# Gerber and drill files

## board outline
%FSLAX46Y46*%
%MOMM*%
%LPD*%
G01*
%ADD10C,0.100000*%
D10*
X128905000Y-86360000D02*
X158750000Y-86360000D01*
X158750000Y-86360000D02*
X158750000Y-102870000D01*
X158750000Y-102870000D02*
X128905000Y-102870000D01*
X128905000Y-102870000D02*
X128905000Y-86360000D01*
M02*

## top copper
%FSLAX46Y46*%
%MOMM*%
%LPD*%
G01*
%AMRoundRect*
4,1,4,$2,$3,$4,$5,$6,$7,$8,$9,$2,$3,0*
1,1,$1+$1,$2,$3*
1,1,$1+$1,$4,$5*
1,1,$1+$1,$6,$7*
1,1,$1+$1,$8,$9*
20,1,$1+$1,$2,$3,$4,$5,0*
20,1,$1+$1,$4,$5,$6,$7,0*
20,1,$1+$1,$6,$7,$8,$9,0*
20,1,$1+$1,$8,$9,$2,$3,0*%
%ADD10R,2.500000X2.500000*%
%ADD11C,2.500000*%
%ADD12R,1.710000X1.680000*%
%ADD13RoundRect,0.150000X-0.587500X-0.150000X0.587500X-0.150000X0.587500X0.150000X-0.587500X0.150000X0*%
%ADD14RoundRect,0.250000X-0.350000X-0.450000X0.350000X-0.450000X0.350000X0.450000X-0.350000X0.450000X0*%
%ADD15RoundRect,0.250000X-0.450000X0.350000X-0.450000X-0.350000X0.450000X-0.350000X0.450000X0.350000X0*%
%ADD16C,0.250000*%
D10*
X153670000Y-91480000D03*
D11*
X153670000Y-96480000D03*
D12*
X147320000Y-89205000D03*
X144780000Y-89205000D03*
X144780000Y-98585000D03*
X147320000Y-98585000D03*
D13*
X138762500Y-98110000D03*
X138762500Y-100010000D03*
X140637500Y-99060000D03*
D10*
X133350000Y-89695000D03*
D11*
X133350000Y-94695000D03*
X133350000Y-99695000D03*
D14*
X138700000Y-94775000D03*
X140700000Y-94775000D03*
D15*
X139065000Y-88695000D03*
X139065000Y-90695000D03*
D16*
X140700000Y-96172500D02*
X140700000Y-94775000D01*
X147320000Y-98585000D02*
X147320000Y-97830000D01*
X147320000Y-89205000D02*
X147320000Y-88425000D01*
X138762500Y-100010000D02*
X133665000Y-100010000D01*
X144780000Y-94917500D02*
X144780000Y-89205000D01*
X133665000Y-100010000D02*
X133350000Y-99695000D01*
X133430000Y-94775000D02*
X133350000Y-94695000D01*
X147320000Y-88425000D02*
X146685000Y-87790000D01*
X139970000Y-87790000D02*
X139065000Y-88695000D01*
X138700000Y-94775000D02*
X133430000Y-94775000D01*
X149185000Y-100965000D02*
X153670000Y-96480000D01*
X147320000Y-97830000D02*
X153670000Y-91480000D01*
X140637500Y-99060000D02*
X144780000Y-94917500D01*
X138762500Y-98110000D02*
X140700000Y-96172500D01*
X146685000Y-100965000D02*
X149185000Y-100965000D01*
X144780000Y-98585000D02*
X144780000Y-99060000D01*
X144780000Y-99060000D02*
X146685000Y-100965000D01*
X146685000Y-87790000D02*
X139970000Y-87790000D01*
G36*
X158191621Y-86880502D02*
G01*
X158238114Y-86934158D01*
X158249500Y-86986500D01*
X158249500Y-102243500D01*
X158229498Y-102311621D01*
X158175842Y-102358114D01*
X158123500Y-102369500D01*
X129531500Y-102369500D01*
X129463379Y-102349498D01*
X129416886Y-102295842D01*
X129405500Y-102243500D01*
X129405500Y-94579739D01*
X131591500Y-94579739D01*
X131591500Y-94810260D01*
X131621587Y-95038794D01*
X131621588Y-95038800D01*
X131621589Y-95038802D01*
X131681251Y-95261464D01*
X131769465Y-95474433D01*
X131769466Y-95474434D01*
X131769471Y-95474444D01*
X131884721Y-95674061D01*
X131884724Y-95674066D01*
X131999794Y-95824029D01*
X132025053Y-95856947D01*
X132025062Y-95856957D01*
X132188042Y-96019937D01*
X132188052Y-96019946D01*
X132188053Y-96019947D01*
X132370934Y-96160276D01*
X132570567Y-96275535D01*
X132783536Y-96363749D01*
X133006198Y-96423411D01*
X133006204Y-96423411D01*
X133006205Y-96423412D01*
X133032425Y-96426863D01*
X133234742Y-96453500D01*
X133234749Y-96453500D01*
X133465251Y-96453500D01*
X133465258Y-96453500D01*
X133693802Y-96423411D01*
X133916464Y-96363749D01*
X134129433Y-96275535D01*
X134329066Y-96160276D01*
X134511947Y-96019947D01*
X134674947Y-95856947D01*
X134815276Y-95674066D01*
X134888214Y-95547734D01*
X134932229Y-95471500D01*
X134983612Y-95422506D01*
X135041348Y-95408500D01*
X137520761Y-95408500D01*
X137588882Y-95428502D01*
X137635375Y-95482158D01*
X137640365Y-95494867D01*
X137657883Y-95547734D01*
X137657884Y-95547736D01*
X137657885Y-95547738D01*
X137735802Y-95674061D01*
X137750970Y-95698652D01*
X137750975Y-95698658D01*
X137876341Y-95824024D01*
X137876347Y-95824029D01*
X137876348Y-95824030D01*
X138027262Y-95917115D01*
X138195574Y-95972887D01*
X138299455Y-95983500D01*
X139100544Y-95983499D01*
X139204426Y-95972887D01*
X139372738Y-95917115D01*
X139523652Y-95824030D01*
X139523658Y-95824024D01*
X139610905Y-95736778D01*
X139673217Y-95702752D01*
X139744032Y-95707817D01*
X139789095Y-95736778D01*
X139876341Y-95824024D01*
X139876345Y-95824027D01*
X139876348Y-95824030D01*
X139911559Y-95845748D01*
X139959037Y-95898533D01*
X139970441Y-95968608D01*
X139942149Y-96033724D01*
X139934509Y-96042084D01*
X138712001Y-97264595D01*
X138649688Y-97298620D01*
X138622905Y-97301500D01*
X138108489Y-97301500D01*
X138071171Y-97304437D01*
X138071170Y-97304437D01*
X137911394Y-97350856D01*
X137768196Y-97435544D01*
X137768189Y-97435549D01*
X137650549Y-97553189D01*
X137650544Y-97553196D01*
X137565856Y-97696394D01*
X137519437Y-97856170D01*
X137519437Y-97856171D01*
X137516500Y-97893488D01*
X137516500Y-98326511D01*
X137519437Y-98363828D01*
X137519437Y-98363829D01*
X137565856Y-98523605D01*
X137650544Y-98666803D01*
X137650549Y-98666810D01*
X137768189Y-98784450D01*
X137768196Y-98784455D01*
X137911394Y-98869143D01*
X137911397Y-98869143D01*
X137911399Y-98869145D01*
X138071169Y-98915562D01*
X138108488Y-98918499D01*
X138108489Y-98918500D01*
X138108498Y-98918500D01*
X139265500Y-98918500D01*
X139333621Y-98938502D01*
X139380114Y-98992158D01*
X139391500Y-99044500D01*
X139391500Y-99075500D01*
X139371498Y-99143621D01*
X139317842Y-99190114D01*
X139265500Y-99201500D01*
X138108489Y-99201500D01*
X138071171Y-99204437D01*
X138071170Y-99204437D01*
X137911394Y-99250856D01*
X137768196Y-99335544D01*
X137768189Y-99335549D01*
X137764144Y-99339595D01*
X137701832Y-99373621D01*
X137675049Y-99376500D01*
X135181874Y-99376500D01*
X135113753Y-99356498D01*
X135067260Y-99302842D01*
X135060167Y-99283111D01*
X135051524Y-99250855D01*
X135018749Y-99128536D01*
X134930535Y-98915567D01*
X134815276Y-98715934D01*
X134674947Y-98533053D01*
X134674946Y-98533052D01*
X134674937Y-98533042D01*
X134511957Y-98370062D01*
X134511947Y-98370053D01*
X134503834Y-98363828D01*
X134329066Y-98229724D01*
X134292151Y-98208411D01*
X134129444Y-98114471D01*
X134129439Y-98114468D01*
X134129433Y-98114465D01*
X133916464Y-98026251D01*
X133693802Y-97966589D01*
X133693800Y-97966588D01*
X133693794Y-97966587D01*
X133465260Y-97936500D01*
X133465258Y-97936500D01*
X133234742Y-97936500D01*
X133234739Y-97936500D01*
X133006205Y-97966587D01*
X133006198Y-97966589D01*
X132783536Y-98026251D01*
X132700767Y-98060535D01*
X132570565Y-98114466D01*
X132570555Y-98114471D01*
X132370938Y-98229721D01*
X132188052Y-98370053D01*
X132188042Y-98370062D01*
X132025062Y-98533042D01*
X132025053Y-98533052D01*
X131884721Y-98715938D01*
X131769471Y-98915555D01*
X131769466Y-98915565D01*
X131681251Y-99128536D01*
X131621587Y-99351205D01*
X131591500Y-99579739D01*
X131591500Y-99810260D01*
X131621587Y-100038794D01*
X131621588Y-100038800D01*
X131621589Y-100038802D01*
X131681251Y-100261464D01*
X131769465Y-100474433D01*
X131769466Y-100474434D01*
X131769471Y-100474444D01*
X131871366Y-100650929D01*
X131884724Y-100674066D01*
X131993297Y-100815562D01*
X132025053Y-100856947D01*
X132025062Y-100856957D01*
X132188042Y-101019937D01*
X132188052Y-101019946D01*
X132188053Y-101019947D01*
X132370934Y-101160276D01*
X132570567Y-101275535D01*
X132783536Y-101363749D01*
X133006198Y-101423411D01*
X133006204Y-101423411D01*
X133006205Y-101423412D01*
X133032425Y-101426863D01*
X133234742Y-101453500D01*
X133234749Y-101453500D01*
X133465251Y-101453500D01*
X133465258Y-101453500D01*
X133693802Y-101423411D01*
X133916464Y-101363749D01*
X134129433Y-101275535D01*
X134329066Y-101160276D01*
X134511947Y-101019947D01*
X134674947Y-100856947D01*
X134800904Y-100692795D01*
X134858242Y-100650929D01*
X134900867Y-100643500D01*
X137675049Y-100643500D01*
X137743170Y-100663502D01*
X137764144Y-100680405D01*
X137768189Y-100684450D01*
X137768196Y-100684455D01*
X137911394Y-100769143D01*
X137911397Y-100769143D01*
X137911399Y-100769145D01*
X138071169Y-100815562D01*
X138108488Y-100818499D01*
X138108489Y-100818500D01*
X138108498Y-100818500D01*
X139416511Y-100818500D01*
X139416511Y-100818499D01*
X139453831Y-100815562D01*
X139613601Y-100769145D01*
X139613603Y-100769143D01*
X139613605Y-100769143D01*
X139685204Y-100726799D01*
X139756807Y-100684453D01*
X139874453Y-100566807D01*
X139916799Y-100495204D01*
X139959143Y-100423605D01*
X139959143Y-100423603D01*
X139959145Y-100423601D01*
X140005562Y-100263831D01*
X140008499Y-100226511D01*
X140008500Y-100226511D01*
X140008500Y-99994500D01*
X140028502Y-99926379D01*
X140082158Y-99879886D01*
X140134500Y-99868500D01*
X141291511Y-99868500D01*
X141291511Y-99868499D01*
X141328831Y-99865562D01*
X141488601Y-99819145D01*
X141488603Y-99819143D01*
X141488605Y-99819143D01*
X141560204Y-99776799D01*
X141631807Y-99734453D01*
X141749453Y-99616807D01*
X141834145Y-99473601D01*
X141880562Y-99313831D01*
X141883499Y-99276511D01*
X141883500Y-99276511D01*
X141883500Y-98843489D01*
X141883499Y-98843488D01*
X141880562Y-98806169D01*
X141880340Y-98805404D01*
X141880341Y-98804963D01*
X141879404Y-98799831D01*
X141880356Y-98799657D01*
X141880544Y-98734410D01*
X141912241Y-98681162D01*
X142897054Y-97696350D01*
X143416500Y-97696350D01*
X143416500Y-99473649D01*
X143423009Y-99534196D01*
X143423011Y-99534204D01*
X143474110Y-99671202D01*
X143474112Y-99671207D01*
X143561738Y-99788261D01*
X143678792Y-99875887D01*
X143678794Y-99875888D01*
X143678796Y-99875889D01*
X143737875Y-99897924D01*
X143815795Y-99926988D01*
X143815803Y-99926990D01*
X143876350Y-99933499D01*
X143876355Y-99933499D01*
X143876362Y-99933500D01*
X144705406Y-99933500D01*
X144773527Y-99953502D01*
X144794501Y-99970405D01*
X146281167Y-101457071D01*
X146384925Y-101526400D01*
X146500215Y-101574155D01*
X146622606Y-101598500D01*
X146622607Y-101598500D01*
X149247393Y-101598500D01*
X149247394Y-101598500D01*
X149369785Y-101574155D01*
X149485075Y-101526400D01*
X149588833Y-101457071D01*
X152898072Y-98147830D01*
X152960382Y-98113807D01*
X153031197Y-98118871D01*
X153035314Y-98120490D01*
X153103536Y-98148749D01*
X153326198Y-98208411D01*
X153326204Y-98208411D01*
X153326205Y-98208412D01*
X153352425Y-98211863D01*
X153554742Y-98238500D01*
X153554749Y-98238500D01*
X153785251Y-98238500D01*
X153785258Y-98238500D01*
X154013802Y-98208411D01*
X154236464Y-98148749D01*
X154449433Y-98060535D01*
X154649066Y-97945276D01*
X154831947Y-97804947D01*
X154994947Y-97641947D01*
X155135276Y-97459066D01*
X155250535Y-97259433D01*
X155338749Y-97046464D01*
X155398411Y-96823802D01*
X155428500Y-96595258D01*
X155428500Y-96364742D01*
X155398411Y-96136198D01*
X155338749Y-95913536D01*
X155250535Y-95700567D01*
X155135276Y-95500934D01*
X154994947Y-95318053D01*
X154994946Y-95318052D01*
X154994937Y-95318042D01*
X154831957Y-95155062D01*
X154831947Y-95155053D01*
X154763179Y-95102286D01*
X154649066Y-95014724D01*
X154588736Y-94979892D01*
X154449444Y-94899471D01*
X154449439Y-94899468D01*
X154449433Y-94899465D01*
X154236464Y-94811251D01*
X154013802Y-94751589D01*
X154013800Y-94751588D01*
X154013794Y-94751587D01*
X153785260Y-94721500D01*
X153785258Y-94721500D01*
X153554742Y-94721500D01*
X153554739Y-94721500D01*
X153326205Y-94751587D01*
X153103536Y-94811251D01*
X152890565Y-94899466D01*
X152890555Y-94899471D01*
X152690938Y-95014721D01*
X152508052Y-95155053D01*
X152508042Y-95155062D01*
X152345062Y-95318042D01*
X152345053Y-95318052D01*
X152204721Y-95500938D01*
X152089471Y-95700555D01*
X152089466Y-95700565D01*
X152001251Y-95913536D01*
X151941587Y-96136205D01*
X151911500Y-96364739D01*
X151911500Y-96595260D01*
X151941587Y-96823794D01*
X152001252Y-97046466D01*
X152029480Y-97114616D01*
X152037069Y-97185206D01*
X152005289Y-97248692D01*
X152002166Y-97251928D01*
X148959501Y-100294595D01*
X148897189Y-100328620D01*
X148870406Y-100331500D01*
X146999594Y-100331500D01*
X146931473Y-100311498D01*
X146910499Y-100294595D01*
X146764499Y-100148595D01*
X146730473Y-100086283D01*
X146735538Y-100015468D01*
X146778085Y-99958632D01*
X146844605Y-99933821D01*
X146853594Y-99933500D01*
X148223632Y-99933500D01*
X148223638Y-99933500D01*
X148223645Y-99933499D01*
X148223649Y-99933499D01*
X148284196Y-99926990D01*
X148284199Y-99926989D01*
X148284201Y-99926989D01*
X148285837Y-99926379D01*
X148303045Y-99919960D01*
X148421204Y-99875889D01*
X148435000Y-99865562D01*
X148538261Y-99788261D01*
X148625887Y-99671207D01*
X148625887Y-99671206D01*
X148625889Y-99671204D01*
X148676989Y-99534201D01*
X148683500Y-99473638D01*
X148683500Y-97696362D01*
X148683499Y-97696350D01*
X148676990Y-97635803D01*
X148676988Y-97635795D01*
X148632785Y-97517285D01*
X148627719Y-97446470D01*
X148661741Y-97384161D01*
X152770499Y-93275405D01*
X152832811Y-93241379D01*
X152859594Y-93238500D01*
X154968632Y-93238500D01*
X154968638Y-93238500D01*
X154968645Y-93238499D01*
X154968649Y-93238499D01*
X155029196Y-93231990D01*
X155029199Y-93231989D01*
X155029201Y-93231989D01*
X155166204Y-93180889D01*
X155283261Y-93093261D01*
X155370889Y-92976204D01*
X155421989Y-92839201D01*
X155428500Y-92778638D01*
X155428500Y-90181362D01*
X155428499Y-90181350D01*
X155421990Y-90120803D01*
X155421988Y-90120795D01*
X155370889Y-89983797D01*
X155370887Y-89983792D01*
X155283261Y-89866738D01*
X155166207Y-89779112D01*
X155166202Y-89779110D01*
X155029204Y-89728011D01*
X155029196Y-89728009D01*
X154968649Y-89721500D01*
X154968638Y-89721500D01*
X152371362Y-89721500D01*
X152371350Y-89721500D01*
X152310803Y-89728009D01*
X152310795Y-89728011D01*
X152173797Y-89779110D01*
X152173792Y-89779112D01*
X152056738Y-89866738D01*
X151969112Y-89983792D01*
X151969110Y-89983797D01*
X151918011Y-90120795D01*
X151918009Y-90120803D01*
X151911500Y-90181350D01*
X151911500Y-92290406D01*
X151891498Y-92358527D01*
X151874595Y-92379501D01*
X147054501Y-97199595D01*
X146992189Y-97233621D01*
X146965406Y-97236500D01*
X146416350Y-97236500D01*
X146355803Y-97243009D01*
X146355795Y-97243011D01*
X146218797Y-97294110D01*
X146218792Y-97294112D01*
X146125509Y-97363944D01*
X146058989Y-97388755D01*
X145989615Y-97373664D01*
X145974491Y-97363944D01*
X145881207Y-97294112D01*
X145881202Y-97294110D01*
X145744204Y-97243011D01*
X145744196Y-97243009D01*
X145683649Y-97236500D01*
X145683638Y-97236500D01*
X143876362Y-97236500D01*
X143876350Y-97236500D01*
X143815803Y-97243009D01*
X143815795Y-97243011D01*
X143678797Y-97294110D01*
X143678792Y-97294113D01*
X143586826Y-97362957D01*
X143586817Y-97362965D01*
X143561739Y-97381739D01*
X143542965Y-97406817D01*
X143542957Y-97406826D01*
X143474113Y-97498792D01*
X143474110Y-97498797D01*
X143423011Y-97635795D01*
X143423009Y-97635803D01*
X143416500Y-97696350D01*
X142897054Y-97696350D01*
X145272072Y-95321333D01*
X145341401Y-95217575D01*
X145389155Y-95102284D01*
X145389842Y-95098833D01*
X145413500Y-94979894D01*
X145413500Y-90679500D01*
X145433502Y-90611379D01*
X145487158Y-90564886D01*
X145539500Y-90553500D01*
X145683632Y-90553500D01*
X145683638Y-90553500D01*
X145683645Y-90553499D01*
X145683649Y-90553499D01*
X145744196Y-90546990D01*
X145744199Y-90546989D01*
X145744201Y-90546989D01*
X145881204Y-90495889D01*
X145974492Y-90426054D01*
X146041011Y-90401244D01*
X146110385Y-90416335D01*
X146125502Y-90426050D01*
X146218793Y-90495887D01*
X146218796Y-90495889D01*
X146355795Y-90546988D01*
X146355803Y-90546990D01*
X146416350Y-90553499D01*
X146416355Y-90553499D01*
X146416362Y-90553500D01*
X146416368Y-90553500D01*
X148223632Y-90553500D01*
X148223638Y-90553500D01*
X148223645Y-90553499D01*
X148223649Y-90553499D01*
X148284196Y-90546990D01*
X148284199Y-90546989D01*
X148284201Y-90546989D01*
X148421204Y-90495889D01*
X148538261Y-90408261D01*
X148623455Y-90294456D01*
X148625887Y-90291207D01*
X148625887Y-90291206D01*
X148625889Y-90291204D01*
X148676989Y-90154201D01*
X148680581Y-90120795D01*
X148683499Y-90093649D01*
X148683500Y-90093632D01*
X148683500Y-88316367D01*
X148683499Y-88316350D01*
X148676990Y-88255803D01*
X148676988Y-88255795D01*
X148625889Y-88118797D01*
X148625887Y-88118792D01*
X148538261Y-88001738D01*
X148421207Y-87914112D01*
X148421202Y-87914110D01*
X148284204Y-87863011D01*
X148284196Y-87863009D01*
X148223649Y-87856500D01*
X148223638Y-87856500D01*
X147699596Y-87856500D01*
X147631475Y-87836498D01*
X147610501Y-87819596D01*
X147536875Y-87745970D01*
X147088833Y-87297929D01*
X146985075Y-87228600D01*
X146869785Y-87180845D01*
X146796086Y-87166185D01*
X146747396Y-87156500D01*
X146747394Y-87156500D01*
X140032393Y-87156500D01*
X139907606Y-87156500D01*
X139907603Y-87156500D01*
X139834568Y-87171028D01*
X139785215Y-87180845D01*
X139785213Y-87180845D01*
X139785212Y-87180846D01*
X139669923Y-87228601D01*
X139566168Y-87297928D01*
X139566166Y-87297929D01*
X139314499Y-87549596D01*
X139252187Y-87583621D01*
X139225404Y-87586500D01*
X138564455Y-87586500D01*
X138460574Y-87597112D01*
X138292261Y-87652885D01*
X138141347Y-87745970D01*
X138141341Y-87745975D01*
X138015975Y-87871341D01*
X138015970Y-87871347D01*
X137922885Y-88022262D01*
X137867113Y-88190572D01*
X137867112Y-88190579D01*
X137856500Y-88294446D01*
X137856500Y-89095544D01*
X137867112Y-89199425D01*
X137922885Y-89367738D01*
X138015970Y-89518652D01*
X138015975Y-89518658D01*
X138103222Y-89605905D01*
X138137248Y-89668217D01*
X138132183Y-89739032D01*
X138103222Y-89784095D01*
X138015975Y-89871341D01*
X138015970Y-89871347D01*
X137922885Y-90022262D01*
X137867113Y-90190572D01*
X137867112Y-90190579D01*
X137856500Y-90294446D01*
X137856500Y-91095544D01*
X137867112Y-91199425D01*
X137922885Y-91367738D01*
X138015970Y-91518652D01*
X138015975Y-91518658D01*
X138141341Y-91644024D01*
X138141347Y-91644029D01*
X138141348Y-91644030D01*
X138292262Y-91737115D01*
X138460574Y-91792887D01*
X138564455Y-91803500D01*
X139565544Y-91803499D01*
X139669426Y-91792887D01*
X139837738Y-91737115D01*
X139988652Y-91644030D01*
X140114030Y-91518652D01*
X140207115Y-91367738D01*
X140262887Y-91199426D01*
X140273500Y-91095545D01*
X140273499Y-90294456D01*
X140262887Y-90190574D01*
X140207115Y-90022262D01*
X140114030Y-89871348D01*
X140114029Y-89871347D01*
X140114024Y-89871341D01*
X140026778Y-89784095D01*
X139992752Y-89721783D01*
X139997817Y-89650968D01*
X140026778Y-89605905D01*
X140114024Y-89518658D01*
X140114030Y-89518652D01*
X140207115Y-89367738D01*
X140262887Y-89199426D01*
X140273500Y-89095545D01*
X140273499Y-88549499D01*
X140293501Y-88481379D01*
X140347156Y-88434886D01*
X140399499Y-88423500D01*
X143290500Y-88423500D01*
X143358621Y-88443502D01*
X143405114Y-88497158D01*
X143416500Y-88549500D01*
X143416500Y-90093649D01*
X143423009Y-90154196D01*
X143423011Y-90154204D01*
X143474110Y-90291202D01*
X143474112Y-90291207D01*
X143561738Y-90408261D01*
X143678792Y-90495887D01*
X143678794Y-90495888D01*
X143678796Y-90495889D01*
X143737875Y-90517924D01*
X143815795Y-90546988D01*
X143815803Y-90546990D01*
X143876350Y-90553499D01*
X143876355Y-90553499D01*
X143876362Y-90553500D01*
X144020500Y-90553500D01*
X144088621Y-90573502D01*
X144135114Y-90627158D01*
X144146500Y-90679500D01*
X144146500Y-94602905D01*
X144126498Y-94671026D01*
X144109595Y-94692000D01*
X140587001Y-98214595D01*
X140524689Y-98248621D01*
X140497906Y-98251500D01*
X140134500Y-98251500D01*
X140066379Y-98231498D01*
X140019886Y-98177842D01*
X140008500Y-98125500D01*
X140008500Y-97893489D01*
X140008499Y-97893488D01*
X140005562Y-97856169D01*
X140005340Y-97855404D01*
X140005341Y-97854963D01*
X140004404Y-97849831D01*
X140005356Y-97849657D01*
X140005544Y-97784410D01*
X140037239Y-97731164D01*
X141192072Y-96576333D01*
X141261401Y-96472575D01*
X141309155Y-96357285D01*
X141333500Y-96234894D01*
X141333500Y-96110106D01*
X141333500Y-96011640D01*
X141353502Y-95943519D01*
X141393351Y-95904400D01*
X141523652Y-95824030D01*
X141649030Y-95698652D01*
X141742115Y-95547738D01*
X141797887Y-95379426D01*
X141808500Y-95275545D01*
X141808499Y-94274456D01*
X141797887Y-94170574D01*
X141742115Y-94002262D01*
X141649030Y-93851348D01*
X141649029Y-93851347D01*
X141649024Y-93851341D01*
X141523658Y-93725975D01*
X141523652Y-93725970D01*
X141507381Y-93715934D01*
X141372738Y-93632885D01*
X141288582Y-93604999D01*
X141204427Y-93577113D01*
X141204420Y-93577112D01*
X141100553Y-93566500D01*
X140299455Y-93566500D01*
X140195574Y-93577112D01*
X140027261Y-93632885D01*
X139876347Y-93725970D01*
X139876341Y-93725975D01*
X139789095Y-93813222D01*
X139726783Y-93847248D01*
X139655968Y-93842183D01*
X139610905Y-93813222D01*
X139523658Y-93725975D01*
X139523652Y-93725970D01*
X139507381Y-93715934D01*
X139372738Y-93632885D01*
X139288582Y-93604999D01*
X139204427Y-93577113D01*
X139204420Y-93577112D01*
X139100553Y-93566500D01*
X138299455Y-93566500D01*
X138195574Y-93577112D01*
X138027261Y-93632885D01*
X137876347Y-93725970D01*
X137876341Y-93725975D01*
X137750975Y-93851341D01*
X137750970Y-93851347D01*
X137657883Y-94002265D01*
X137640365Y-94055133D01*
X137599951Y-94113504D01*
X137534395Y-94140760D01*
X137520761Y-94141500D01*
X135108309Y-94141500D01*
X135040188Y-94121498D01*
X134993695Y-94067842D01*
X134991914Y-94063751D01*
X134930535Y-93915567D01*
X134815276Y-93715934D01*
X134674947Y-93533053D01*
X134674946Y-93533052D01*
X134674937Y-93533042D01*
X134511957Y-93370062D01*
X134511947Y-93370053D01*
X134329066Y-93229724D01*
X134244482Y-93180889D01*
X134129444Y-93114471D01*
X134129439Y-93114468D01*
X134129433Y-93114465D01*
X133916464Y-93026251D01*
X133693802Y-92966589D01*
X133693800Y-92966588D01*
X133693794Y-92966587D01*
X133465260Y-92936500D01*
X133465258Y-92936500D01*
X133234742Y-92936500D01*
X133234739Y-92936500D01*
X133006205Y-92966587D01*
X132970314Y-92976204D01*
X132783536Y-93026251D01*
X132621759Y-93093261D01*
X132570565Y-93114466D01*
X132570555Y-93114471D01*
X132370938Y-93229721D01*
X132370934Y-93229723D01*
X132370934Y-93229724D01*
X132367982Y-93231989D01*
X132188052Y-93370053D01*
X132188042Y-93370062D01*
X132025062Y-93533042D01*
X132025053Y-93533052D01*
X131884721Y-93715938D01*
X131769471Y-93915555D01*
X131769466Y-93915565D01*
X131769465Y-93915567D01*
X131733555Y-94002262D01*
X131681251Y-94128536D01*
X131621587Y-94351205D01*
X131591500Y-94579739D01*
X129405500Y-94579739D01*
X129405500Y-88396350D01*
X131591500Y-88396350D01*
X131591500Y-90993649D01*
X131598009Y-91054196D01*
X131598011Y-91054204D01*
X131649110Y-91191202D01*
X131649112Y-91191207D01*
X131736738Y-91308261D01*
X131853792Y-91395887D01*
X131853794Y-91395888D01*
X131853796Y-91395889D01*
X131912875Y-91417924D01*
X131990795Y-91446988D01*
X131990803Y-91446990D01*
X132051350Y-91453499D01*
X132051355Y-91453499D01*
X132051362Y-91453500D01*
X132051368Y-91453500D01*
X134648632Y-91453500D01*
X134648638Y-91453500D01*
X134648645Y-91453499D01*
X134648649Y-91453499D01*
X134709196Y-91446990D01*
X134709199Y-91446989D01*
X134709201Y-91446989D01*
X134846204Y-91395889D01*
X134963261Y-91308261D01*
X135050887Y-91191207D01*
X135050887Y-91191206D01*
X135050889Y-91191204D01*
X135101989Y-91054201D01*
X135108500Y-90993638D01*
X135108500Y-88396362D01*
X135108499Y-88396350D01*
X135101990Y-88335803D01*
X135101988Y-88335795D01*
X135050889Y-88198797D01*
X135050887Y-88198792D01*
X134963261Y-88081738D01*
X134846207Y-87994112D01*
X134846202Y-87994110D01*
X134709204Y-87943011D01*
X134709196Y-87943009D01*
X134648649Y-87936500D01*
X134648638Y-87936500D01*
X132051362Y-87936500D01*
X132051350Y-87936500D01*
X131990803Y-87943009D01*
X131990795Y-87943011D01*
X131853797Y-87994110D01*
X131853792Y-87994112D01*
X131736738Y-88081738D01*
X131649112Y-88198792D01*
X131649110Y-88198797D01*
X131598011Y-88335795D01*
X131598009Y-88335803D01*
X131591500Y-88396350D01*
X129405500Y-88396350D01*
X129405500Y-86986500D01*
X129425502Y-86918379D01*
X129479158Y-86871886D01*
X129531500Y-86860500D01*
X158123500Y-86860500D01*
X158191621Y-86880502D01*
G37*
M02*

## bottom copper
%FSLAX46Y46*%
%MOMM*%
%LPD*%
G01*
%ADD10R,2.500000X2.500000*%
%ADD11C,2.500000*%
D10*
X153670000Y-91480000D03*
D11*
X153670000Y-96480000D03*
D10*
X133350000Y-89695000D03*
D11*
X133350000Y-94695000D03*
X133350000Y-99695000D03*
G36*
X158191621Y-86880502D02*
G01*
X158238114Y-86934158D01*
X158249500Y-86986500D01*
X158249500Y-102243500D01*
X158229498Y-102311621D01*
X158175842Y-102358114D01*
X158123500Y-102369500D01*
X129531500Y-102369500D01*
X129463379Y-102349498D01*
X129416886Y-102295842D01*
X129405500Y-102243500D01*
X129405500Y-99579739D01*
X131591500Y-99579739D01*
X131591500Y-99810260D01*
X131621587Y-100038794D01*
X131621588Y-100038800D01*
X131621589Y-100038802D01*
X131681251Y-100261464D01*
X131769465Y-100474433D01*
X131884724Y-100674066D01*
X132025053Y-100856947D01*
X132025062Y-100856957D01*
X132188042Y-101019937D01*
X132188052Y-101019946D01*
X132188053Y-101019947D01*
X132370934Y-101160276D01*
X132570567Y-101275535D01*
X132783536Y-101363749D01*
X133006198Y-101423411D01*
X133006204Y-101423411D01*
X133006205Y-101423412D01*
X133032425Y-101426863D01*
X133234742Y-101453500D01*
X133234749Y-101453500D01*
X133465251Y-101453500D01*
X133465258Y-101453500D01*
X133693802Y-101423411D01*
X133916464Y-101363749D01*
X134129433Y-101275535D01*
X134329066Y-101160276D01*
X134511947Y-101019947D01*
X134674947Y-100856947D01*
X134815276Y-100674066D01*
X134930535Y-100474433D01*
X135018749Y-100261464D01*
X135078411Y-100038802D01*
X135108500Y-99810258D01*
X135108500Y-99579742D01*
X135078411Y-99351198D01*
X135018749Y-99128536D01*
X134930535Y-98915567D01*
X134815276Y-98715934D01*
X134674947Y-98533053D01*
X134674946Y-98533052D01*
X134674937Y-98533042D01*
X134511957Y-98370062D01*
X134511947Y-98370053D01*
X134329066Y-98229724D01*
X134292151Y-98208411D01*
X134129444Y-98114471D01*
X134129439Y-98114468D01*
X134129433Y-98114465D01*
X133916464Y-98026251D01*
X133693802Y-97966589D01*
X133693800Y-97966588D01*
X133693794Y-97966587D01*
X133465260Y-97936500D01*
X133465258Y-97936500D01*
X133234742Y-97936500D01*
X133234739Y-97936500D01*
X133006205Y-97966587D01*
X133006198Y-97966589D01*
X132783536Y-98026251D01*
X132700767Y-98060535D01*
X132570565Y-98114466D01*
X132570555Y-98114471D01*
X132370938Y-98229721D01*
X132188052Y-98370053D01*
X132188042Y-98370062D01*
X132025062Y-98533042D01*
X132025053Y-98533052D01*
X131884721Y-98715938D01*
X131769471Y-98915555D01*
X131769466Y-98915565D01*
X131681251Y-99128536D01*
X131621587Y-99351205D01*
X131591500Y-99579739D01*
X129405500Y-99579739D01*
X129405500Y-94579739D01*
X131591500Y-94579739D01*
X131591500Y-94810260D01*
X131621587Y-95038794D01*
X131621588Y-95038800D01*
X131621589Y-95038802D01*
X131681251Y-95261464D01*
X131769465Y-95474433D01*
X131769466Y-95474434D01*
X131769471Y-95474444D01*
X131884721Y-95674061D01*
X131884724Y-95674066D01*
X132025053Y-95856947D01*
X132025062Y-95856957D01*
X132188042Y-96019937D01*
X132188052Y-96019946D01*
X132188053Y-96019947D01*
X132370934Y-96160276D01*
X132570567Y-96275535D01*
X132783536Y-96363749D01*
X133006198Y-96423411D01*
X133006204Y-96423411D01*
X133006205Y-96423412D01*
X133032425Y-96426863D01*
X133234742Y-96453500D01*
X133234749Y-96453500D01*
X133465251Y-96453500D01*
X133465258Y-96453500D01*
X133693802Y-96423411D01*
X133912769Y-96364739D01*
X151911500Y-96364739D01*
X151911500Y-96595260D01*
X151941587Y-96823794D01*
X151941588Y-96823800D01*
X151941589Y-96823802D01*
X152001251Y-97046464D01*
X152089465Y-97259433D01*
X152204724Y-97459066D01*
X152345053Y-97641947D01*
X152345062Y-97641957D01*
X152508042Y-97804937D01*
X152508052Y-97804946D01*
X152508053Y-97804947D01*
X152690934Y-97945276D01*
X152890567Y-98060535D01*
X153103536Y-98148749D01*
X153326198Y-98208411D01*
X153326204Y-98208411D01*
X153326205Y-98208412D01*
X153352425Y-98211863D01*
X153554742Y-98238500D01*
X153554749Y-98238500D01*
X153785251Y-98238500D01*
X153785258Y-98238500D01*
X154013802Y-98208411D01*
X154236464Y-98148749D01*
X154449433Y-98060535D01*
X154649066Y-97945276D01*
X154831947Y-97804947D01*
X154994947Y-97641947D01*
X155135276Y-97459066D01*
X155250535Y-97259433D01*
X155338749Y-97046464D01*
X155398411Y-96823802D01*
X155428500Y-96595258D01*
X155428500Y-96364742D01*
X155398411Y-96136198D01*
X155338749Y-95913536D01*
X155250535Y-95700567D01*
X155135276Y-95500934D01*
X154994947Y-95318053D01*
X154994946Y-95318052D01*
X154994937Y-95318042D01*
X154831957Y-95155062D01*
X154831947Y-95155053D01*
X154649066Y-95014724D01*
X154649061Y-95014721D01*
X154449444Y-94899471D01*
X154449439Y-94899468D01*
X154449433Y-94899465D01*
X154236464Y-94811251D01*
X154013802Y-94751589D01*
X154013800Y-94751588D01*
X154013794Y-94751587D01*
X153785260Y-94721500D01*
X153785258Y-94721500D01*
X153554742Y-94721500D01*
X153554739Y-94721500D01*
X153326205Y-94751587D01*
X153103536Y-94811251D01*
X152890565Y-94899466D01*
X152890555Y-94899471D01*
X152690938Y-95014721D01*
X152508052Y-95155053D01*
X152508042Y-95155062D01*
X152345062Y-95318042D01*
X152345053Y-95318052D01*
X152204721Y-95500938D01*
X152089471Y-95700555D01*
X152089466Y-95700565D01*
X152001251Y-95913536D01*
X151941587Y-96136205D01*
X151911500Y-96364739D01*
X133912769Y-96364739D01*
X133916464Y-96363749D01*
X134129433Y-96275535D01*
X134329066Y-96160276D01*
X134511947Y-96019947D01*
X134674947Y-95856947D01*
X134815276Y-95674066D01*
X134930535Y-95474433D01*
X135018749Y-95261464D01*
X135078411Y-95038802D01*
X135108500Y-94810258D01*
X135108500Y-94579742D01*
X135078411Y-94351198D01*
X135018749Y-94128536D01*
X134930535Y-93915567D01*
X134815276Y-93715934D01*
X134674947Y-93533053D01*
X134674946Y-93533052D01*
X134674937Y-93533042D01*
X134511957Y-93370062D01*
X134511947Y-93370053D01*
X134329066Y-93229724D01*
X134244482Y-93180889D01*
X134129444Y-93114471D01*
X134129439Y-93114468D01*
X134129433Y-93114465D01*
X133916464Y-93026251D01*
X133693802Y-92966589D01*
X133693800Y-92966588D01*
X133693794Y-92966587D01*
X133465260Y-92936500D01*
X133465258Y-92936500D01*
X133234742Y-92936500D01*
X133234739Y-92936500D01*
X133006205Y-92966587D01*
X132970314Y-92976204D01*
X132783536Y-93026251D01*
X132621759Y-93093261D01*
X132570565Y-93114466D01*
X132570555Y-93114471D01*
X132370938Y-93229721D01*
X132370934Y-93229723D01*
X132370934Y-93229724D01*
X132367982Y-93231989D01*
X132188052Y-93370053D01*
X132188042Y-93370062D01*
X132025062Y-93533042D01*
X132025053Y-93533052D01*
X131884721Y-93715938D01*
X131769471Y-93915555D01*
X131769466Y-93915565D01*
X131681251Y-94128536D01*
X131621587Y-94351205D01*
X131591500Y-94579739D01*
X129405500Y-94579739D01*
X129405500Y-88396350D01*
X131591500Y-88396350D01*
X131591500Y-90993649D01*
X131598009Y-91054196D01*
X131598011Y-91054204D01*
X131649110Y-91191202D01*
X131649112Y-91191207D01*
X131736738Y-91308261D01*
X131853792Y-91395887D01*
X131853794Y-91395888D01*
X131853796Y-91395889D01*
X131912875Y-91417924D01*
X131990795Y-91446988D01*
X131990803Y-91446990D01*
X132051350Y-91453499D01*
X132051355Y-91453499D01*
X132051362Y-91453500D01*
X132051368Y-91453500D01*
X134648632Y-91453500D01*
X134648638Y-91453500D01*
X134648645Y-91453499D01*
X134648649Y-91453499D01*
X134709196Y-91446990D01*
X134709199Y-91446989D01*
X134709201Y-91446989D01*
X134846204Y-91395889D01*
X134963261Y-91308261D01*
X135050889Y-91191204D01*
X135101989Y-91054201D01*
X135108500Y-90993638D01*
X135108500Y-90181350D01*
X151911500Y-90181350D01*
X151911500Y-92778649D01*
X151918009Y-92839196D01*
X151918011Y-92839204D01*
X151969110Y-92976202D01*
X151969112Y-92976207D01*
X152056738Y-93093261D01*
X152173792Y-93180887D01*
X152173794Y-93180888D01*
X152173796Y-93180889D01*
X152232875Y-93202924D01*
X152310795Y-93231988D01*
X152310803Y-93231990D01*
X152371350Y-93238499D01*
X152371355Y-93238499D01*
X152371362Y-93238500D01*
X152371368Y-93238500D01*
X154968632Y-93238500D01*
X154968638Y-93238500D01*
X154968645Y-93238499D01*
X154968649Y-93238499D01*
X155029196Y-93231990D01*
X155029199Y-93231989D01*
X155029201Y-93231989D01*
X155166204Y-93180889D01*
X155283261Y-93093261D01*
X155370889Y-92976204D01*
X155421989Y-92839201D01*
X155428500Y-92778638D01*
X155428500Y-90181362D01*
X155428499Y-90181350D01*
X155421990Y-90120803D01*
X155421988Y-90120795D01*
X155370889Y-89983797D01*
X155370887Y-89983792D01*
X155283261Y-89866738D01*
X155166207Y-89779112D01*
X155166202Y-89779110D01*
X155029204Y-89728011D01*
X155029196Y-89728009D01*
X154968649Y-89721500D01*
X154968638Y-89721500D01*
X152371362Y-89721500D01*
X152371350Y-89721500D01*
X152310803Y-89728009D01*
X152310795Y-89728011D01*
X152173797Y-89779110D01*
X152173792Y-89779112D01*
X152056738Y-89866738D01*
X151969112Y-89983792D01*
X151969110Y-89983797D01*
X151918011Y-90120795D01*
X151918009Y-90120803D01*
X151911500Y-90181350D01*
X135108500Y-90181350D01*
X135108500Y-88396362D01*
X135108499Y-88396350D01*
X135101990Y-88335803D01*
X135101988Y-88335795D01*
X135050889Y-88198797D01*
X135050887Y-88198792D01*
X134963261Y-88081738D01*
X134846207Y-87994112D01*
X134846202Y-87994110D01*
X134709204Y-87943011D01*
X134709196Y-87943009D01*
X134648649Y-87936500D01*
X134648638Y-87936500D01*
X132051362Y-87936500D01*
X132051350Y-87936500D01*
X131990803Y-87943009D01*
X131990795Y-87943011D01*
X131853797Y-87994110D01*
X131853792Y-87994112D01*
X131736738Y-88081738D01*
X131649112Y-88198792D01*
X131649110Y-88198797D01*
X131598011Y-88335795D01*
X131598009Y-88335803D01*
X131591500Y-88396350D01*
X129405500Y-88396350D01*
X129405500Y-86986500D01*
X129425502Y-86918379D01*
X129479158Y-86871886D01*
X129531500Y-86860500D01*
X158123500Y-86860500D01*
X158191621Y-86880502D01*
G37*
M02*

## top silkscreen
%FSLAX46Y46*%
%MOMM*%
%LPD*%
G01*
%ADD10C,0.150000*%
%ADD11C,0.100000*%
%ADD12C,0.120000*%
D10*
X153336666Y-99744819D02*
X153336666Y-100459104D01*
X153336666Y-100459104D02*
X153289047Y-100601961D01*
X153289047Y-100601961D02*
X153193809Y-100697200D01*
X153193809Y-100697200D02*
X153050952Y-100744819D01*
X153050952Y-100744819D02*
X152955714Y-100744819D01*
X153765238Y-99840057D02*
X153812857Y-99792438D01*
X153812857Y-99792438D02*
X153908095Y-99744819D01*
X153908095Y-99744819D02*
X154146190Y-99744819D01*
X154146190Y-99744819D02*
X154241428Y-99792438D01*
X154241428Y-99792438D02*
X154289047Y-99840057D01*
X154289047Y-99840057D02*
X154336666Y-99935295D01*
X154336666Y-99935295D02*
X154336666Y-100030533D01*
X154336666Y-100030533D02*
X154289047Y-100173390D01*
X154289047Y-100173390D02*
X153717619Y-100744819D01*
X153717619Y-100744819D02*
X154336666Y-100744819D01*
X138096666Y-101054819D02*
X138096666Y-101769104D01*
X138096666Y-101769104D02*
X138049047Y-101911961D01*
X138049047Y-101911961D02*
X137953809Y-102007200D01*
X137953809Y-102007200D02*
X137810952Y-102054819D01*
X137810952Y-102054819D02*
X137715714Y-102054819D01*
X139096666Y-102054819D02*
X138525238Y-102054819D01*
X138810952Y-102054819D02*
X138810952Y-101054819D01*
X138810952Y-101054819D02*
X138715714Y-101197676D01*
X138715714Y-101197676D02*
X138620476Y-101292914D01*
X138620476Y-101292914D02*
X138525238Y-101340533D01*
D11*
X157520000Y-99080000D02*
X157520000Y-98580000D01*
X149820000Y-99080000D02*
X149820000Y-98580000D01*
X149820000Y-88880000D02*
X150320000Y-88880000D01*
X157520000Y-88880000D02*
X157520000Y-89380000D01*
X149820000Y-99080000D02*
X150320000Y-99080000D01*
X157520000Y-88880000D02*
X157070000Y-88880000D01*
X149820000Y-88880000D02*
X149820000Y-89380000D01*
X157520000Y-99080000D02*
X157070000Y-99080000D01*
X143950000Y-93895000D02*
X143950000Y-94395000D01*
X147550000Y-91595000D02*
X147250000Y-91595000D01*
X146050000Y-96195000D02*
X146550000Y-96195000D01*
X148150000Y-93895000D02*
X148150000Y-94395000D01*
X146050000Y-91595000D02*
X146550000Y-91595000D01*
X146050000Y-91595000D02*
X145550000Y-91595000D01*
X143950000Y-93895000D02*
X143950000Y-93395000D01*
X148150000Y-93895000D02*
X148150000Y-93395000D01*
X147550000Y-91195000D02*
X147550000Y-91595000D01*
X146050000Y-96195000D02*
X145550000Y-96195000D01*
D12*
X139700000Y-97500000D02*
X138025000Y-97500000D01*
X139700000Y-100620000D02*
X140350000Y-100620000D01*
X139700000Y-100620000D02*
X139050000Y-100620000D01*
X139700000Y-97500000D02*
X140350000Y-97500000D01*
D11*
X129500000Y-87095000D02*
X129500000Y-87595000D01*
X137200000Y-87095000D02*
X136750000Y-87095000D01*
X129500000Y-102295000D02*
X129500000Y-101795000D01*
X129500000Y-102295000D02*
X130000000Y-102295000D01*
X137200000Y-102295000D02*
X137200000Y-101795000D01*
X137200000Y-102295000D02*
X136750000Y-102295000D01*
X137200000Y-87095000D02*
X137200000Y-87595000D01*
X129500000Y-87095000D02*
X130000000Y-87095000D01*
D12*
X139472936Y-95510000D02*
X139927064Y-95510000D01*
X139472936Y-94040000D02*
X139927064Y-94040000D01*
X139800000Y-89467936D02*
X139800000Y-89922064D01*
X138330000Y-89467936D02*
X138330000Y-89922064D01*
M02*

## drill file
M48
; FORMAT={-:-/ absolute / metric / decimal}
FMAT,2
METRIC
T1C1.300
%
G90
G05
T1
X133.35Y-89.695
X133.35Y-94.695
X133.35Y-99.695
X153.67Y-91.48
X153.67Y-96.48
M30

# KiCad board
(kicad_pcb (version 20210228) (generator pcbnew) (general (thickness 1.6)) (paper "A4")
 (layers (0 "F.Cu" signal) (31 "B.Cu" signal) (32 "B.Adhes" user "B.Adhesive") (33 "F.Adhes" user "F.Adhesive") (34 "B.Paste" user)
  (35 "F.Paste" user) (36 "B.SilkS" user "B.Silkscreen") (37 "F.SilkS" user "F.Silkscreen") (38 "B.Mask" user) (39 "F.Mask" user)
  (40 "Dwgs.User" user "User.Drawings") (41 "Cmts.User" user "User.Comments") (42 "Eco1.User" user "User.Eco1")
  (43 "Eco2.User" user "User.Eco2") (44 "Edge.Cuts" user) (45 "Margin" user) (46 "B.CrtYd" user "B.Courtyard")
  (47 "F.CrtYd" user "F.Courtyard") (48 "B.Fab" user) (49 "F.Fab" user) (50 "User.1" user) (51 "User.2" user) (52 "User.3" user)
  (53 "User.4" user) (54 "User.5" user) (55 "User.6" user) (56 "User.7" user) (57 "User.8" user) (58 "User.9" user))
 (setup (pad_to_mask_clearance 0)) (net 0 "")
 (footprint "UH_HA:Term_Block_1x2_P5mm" (layer "F.Cu") (at 153.67 91.48 -90)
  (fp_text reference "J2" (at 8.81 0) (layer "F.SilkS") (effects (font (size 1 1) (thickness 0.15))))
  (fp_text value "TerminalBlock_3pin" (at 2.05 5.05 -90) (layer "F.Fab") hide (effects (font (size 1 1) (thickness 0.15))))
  (fp_line (start 7.6 -3.85) (end 7.1 -3.85) (layer "F.SilkS") (width 0.1))
  (fp_line (start 7.6 3.85) (end 7.1 3.85) (layer "F.SilkS") (width 0.1))
  (fp_line (start -2.6 3.85) (end -2.6 3.35) (layer "F.SilkS") (width 0.1))
  (fp_line (start -2.6 -3.85) (end -2.1 -3.85) (layer "F.SilkS") (width 0.1))
  (fp_line (start 7.6 3.85) (end 7.6 3.35) (layer "F.SilkS") (width 0.1))
  (fp_line (start -2.6 -3.85) (end -2.6 -3.4) (layer "F.SilkS") (width 0.1))
  (fp_line (start -2.6 3.85) (end -2.1 3.85) (layer "F.SilkS") (width 0.1))
  (fp_line (start 7.6 -3.85) (end 7.6 -3.4) (layer "F.SilkS") (width 0.1))
  (pad "1" thru_hole rect (at 0 0 270) (locked) (size 2.5 2.5) (drill 1.3) (layers *.Cu *.Mask))
  (pad "2" thru_hole circle (at 5 0 270) (locked) (size 2.5 2.5) (drill 1.3) (layers *.Cu *.Mask)))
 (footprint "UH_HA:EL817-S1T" (layer "F.Cu") (at 146.05 93.895 -90)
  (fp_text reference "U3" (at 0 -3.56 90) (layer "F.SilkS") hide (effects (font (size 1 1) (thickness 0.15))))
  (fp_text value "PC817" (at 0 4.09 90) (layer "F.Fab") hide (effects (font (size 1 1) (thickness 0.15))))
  (fp_line (start 0 2.1) (end 0.5 2.1) (layer "F.SilkS") (width 0.1))
  (fp_line (start -2.3 -1.5) (end -2.3 -1.2) (layer "F.SilkS") (width 0.1))
  (fp_line (start 2.3 0) (end 2.3 -0.5) (layer "F.SilkS") (width 0.1))
  (fp_line (start 0 -2.1) (end 0.5 -2.1) (layer "F.SilkS") (width 0.1))
  (fp_line (start -2.3 0) (end -2.3 -0.5) (layer "F.SilkS") (width 0.1))
  (fp_line (start -2.3 0) (end -2.3 0.5) (layer "F.SilkS") (width 0.1))
  (fp_line (start 0 2.1) (end -0.5 2.1) (layer "F.SilkS") (width 0.1))
  (fp_line (start 0 -2.1) (end -0.5 -2.1) (layer "F.SilkS") (width 0.1))
  (fp_line (start -2.7 -1.5) (end -2.3 -1.5) (layer "F.SilkS") (width 0.1))
  (fp_line (start 2.3 0) (end 2.3 0.5) (layer "F.SilkS") (width 0.1))
  (pad "1" smd rect (at -4.69 -1.27 270) (locked) (size 1.68 1.71) (layers "F.Cu" "F.Paste" "F.Mask"))
  (pad "2" smd rect (at -4.69 1.27 270) (locked) (size 1.68 1.71) (layers "F.Cu" "F.Paste" "F.Mask"))
  (pad "3" smd rect (at 4.69 1.27 270) (locked) (size 1.68 1.71) (layers "F.Cu" "F.Paste" "F.Mask"))
  (pad "4" smd rect (at 4.69 -1.27 270) (locked) (size 1.68 1.71) (layers "F.Cu" "F.Paste" "F.Mask")))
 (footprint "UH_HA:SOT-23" (layer "F.Cu") (at 139.7 99.06)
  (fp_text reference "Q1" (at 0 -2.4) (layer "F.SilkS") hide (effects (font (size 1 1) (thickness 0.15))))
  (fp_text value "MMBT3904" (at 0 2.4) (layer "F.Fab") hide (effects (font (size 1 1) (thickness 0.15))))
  (fp_line (start 0 -1.56) (end -1.675 -1.56) (layer "F.SilkS") (width 0.12))
  (fp_line (start 0 1.56) (end 0.65 1.56) (layer "F.SilkS") (width 0.12))
  (fp_line (start 0 1.56) (end -0.65 1.56) (layer "F.SilkS") (width 0.12))
  (fp_line (start 0 -1.56) (end 0.65 -1.56) (layer "F.SilkS") (width 0.12))
  (pad "1" smd roundrect (at -0.9375 -0.95) (locked) (size 1.475 0.6) (layers "F.Cu" "F.Paste" "F.Mask") (roundrect_rratio 0.25))
  (pad "2" smd roundrect (at -0.9375 0.95) (locked) (size 1.475 0.6) (layers "F.Cu" "F.Paste" "F.Mask") (roundrect_rratio 0.25))
  (pad "3" smd roundrect (at 0.9375 0) (locked) (size 1.475 0.6) (layers "F.Cu" "F.Paste" "F.Mask") (roundrect_rratio 0.25)))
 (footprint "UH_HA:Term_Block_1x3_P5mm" (layer "F.Cu") (at 133.35 89.695 -90)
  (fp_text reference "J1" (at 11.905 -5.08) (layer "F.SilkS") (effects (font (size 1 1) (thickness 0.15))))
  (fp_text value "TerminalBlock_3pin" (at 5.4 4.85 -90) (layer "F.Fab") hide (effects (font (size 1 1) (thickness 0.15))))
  (fp_line (start -2.6 3.85) (end -2.1 3.85) (layer "F.SilkS") (width 0.1))
  (fp_line (start -2.6 -3.85) (end -2.6 -3.4) (layer "F.SilkS") (width 0.1))
  (fp_line (start 12.6 3.85) (end 12.1 3.85) (layer "F.SilkS") (width 0.1))
  (fp_line (start 12.6 3.85) (end 12.6 3.35) (layer "F.SilkS") (width 0.1))
  (fp_line (start 12.6 -3.85) (end 12.1 -3.85) (layer "F.SilkS") (width 0.1))
  (fp_line (start 12.6 -3.85) (end 12.6 -3.4) (layer "F.SilkS") (width 0.1))
  (fp_line (start -2.6 -3.85) (end -2.1 -3.85) (layer "F.SilkS") (width 0.1))
  (fp_line (start -2.6 3.85) (end -2.6 3.35) (layer "F.SilkS") (width 0.1))
  (pad "1" thru_hole rect (at 0 0 270) (locked) (size 2.5 2.5) (drill 1.3) (layers *.Cu *.Mask))
  (pad "2" thru_hole circle (at 5 0 270) (locked) (size 2.5 2.5) (drill 1.3) (layers *.Cu *.Mask))
  (pad "3" thru_hole circle (at 10 0 270) (locked) (size 2.5 2.5) (drill 1.3) (layers *.Cu *.Mask)))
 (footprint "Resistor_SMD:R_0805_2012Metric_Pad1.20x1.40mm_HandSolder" (layer "F.Cu") (at 139.7 94.775)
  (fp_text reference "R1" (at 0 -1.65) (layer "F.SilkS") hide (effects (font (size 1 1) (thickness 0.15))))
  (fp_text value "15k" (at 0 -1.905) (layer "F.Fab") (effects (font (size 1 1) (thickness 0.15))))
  (fp_line (start -0.227064 0.735) (end 0.227064 0.735) (layer "F.SilkS") (width 0.12))
  (fp_line (start -0.227064 -0.735) (end 0.227064 -0.735) (layer "F.SilkS") (width 0.12))
  (pad "1" smd roundrect (at -1 0) (locked) (size 1.2 1.4) (layers "F.Cu" "F.Paste" "F.Mask") (roundrect_rratio 0.208333))
  (pad "2" smd roundrect (at 1 0) (locked) (size 1.2 1.4) (layers "F.Cu" "F.Paste" "F.Mask") (roundrect_rratio 0.208333)))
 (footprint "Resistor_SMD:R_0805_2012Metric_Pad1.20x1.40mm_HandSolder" (layer "F.Cu") (at 139.065 89.695 -90)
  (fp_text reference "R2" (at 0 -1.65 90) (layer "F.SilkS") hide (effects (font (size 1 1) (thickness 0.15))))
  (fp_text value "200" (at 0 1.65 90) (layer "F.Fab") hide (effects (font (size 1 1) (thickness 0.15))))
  (fp_line (start -0.227064 -0.735) (end 0.227064 -0.735) (layer "F.SilkS") (width 0.12))
  (fp_line (start -0.227064 0.735) (end 0.227064 0.735) (layer "F.SilkS") (width 0.12))
  (pad "1" smd roundrect (at -1 0 270) (locked) (size 1.2 1.4) (layers "F.Cu" "F.Paste" "F.Mask") (roundrect_rratio 0.208333))
  (pad "2" smd roundrect (at 1 0 270) (locked) (size 1.2 1.4) (layers "F.Cu" "F.Paste" "F.Mask") (roundrect_rratio 0.208333)))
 (gr_line (start 128.905 86.36) (end 158.75 86.36) (layer "Edge.Cuts") (width 0.1))
 (gr_line (start 158.75 86.36) (end 158.75 102.87) (layer "Edge.Cuts") (width 0.1))
 (gr_line (start 158.75 102.87) (end 128.905 102.87) (layer "Edge.Cuts") (width 0.1))
 (gr_line (start 128.905 102.87) (end 128.905 86.36) (layer "Edge.Cuts") (width 0.1))
 (segment (start 140.7 96.1725) (end 140.7 94.775) (width 0.25) (layer "F.Cu") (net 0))
 (segment (start 147.32 98.585) (end 147.32 97.83) (width 0.25) (layer "F.Cu") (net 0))
 (segment (start 147.32 89.205) (end 147.32 88.425) (width 0.25) (layer "F.Cu") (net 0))
 (segment (start 138.7625 100.01) (end 133.665 100.01) (width 0.25) (layer "F.Cu") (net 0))
 (segment (start 144.78 94.9175) (end 144.78 89.205) (width 0.25) (layer "F.Cu") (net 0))
 (segment (start 133.665 100.01) (end 133.35 99.695) (width 0.25) (layer "F.Cu") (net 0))
 (segment (start 133.43 94.775) (end 133.35 94.695) (width 0.25) (layer "F.Cu") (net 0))
 (segment (start 147.32 88.425) (end 146.685 87.79) (width 0.25) (layer "F.Cu") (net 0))
 (segment (start 139.97 87.79) (end 139.065 88.695) (width 0.25) (layer "F.Cu") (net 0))
 (segment (start 138.7 94.775) (end 133.43 94.775) (width 0.25) (layer "F.Cu") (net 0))
 (segment (start 149.185 100.965) (end 153.67 96.48) (width 0.25) (layer "F.Cu") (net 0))
 (segment (start 147.32 97.83) (end 153.67 91.48) (width 0.25) (layer "F.Cu") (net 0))
 (segment (start 140.6375 99.06) (end 144.78 94.9175) (width 0.25) (layer "F.Cu") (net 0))
 (segment (start 138.7625 98.11) (end 140.7 96.1725) (width 0.25) (layer "F.Cu") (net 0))
 (segment (start 146.685 100.965) (end 149.185 100.965) (width 0.25) (layer "F.Cu") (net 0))
 (segment (start 144.78 98.585) (end 144.78 99.06) (width 0.25) (layer "F.Cu") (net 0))
 (segment (start 144.78 99.06) (end 146.685 100.965) (width 0.25) (layer "F.Cu") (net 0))
 (segment (start 146.685 87.79) (end 139.97 87.79) (width 0.25) (layer "F.Cu") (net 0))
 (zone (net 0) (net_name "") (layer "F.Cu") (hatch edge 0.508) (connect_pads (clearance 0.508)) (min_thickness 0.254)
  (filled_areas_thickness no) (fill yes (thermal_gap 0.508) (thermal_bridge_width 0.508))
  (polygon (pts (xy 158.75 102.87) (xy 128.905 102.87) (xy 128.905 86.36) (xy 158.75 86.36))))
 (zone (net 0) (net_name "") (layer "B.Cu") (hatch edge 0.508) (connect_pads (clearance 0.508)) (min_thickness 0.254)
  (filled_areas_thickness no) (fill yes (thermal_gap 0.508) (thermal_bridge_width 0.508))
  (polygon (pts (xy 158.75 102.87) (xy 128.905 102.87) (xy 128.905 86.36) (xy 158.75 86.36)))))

